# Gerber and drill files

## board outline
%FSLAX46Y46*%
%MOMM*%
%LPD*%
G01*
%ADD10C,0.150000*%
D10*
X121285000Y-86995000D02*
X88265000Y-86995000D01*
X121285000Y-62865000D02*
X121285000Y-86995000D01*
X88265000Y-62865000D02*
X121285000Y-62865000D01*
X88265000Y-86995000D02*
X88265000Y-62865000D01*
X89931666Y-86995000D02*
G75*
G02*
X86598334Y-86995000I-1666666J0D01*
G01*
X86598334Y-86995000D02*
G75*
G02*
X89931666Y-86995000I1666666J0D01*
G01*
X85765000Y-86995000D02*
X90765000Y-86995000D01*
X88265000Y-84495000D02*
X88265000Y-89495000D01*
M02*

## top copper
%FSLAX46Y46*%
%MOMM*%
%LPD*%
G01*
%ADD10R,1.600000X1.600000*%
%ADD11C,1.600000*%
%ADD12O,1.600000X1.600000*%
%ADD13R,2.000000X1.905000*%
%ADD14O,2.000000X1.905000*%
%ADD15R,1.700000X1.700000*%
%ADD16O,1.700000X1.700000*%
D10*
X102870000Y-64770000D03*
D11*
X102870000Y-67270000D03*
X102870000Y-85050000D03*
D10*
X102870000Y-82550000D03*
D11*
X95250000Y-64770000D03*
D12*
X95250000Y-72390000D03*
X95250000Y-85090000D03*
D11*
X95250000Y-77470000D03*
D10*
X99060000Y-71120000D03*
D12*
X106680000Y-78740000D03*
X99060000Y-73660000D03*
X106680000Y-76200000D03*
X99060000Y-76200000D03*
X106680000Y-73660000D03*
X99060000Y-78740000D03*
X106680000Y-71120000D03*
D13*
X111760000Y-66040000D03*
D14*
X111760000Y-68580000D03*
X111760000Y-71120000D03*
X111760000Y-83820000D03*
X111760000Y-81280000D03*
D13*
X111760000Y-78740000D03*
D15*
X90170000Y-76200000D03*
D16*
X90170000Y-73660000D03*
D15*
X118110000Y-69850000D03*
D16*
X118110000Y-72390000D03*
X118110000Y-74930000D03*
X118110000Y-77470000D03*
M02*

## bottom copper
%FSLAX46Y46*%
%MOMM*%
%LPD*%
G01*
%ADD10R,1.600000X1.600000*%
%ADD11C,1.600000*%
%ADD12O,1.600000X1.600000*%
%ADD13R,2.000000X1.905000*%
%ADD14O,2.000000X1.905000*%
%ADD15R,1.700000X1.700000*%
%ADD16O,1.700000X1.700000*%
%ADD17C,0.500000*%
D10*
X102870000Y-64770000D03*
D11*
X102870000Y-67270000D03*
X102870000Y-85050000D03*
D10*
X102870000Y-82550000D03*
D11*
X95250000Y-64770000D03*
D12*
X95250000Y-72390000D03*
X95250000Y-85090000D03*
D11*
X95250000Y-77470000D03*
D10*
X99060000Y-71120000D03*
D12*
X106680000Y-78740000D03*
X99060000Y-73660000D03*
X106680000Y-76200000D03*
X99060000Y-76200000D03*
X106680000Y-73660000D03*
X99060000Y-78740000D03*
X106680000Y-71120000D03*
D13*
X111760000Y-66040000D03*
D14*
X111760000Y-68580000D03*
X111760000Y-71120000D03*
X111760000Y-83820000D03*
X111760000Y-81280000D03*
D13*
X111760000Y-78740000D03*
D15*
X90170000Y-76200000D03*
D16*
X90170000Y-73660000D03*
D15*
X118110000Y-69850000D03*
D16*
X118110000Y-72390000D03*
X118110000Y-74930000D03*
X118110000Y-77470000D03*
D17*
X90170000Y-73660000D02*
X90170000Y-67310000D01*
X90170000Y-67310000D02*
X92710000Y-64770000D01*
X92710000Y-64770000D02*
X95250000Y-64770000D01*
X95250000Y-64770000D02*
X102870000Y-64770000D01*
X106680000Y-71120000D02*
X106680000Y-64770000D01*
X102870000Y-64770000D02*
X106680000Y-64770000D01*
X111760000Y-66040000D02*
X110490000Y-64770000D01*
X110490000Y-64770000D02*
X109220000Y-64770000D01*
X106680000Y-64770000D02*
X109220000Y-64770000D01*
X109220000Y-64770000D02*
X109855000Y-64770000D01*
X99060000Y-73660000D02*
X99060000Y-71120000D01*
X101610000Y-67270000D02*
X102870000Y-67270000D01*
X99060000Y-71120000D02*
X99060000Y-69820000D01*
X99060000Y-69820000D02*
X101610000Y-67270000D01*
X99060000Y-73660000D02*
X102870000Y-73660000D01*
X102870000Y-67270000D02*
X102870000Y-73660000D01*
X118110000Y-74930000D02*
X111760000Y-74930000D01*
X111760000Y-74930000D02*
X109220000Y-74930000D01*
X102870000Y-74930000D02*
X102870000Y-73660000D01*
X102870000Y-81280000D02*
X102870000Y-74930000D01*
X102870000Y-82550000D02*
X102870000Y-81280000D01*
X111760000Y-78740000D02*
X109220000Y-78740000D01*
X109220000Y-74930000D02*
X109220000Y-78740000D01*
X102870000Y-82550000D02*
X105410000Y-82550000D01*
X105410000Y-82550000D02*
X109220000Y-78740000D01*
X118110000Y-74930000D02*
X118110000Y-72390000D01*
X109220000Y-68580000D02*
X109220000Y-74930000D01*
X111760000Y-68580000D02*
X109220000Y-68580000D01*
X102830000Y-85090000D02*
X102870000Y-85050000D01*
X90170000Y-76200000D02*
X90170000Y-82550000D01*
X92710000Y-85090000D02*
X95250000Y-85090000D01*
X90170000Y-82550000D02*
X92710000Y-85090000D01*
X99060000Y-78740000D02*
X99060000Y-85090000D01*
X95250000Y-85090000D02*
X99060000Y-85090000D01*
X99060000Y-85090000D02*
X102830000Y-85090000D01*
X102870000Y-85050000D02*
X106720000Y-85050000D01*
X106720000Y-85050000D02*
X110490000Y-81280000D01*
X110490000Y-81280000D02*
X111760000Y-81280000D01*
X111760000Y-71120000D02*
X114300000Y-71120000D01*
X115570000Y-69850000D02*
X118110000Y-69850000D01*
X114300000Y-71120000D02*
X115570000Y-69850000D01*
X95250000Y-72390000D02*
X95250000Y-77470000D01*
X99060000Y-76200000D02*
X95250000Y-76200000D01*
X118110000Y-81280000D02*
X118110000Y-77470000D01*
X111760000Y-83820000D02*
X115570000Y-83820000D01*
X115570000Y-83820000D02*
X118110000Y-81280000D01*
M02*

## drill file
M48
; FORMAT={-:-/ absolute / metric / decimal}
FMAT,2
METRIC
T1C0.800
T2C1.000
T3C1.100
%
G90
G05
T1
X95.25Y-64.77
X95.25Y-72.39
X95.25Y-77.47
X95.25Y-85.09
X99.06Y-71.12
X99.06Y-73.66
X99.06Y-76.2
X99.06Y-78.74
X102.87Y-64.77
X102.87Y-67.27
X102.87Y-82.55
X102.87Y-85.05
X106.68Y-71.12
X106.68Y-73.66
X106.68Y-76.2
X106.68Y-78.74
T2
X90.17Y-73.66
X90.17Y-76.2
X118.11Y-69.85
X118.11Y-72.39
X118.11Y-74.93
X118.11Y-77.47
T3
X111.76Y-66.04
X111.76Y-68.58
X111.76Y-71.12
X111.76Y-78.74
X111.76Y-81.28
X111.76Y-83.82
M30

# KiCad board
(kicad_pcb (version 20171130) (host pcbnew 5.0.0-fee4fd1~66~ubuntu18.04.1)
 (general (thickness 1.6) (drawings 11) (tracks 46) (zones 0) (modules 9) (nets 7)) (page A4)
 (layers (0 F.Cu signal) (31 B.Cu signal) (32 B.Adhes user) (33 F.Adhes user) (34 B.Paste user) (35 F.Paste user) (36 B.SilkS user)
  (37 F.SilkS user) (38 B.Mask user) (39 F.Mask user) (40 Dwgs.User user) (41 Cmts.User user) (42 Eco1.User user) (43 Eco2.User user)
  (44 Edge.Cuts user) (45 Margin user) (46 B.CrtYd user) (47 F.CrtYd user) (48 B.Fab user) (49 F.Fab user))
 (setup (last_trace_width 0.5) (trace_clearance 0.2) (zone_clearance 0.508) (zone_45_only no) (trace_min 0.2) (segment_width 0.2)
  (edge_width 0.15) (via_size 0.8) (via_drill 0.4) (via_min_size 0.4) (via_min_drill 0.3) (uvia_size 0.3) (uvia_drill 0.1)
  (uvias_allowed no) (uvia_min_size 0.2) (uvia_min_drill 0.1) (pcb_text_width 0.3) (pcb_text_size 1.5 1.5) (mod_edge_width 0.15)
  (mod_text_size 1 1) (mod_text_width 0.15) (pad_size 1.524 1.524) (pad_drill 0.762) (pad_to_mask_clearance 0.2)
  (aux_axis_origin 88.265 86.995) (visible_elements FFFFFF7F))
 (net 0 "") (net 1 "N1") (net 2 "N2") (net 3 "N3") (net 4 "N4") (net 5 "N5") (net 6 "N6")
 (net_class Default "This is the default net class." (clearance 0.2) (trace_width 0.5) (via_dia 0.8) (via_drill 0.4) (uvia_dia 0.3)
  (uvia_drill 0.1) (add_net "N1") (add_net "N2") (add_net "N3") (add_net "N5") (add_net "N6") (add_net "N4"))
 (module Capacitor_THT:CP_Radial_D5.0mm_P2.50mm (layer F.Cu) (at 102.87 64.77 270)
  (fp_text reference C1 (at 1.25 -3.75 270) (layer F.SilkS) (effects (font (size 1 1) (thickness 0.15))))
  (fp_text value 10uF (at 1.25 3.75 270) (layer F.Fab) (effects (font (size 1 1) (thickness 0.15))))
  (pad 1 thru_hole rect (at 0 0 270) (size 1.6 1.6) (drill 0.8) (layers *.Cu *.Mask) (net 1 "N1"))
  (pad 2 thru_hole circle (at 2.5 0 270) (size 1.6 1.6) (drill 0.8) (layers *.Cu *.Mask) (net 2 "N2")))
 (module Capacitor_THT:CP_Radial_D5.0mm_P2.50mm (layer F.Cu) (at 102.87 82.55 270)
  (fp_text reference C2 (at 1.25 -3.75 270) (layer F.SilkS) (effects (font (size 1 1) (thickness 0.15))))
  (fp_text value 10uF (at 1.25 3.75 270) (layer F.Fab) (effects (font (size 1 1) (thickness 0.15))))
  (pad 2 thru_hole circle (at 2.5 0 270) (size 1.6 1.6) (drill 0.8) (layers *.Cu *.Mask) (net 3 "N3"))
  (pad 1 thru_hole rect (at 0 0 270) (size 1.6 1.6) (drill 0.8) (layers *.Cu *.Mask) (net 2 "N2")))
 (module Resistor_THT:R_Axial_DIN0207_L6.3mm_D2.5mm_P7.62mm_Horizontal (layer F.Cu) (at 95.25 64.77 270)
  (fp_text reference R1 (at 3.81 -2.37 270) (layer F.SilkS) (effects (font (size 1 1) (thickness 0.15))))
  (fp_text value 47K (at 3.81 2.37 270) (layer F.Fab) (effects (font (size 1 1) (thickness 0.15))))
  (pad 1 thru_hole circle (at 0 0 270) (size 1.6 1.6) (drill 0.8) (layers *.Cu *.Mask) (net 1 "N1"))
  (pad 2 thru_hole oval (at 7.62 0 270) (size 1.6 1.6) (drill 0.8) (layers *.Cu *.Mask) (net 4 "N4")))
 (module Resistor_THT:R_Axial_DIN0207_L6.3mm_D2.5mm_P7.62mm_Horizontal (layer F.Cu) (at 95.25 77.47 270)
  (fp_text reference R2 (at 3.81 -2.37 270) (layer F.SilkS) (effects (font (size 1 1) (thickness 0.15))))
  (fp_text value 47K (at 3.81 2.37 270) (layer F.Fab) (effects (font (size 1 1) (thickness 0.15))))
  (pad 2 thru_hole oval (at 7.62 0 270) (size 1.6 1.6) (drill 0.8) (layers *.Cu *.Mask) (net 3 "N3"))
  (pad 1 thru_hole circle (at 0 0 270) (size 1.6 1.6) (drill 0.8) (layers *.Cu *.Mask) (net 4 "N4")))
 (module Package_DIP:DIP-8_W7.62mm (layer F.Cu) (at 99.06 71.12)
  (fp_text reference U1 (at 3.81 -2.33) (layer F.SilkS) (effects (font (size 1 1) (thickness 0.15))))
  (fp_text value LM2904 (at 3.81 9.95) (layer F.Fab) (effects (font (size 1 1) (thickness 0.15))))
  (pad 1 thru_hole rect (at 0 0) (size 1.6 1.6) (drill 0.8) (layers *.Cu *.Mask) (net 2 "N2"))
  (pad 5 thru_hole oval (at 7.62 7.62) (size 1.6 1.6) (drill 0.8) (layers *.Cu *.Mask))
  (pad 2 thru_hole oval (at 0 2.54) (size 1.6 1.6) (drill 0.8) (layers *.Cu *.Mask) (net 2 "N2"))
  (pad 6 thru_hole oval (at 7.62 5.08) (size 1.6 1.6) (drill 0.8) (layers *.Cu *.Mask))
  (pad 3 thru_hole oval (at 0 5.08) (size 1.6 1.6) (drill 0.8) (layers *.Cu *.Mask) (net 4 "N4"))
  (pad 7 thru_hole oval (at 7.62 2.54) (size 1.6 1.6) (drill 0.8) (layers *.Cu *.Mask))
  (pad 4 thru_hole oval (at 0 7.62) (size 1.6 1.6) (drill 0.8) (layers *.Cu *.Mask) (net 3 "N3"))
  (pad 8 thru_hole oval (at 7.62 0) (size 1.6 1.6) (drill 0.8) (layers *.Cu *.Mask) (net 1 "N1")))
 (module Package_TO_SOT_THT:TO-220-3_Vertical (layer F.Cu) (at 111.76 66.04 270)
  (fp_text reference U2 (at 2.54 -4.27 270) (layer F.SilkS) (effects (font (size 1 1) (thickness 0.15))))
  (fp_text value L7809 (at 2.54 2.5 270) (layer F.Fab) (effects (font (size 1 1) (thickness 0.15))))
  (pad 1 thru_hole rect (at 0 0 270) (size 1.905 2) (drill 1.1) (layers *.Cu *.Mask) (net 1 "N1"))
  (pad 2 thru_hole oval (at 2.54 0 270) (size 1.905 2) (drill 1.1) (layers *.Cu *.Mask) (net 2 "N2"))
  (pad 3 thru_hole oval (at 5.08 0 270) (size 1.905 2) (drill 1.1) (layers *.Cu *.Mask) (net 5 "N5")))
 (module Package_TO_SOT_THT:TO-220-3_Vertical (layer F.Cu) (at 111.76 78.74 270)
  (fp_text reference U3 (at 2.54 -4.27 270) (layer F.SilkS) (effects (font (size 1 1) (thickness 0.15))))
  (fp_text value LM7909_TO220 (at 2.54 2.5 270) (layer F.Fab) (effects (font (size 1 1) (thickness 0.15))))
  (pad 3 thru_hole oval (at 5.08 0 270) (size 1.905 2) (drill 1.1) (layers *.Cu *.Mask) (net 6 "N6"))
  (pad 2 thru_hole oval (at 2.54 0 270) (size 1.905 2) (drill 1.1) (layers *.Cu *.Mask) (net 3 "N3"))
  (pad 1 thru_hole rect (at 0 0 270) (size 1.905 2) (drill 1.1) (layers *.Cu *.Mask) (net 2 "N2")))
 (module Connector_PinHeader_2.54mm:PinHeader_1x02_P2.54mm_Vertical (layer F.Cu) (at 90.17 76.2 180)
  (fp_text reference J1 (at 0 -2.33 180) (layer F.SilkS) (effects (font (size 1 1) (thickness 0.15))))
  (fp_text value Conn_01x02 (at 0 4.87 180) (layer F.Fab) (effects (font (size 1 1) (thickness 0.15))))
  (pad 1 thru_hole rect (at 0 0 180) (size 1.7 1.7) (drill 1) (layers *.Cu *.Mask) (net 3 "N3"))
  (pad 2 thru_hole oval (at 0 2.54 180) (size 1.7 1.7) (drill 1) (layers *.Cu *.Mask) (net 1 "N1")))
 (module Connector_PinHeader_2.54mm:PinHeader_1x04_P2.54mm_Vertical (layer F.Cu) (at 118.11 69.85)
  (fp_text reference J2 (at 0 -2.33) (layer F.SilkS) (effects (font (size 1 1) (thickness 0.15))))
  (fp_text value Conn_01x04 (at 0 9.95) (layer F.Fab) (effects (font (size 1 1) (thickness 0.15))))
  (pad 1 thru_hole rect (at 0 0) (size 1.7 1.7) (drill 1) (layers *.Cu *.Mask) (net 5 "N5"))
  (pad 2 thru_hole oval (at 0 2.54) (size 1.7 1.7) (drill 1) (layers *.Cu *.Mask) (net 2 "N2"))
  (pad 3 thru_hole oval (at 0 5.08) (size 1.7 1.7) (drill 1) (layers *.Cu *.Mask) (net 2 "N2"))
  (pad 4 thru_hole oval (at 0 7.62) (size 1.7 1.7) (drill 1) (layers *.Cu *.Mask) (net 6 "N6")))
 (gr_line (start 121.285 86.995) (end 88.265 86.995) (layer Edge.Cuts) (width 0.15))
 (gr_line (start 121.285 62.865) (end 121.285 86.995) (layer Edge.Cuts) (width 0.15))
 (gr_line (start 88.265 62.865) (end 121.285 62.865) (layer Edge.Cuts) (width 0.15))
 (gr_line (start 88.265 86.995) (end 88.265 62.865) (layer Edge.Cuts) (width 0.15))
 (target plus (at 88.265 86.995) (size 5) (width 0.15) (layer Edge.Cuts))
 (segment (start 90.17 73.66) (end 90.17 67.31) (width 0.5) (layer B.Cu) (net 1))
 (segment (start 90.17 67.31) (end 92.71 64.77) (width 0.5) (layer B.Cu) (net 1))
 (segment (start 92.71 64.77) (end 95.25 64.77) (width 0.5) (layer B.Cu) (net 1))
 (segment (start 95.25 64.77) (end 102.87 64.77) (width 0.5) (layer B.Cu) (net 1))
 (segment (start 106.68 71.12) (end 106.68 64.77) (width 0.5) (layer B.Cu) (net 1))
 (segment (start 102.87 64.77) (end 106.68 64.77) (width 0.5) (layer B.Cu) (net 1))
 (segment (start 111.76 66.04) (end 110.49 64.77) (width 0.5) (layer B.Cu) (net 1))
 (segment (start 110.49 64.77) (end 109.22 64.77) (width 0.5) (layer B.Cu) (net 1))
 (segment (start 106.68 64.77) (end 109.22 64.77) (width 0.5) (layer B.Cu) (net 1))
 (segment (start 109.22 64.77) (end 109.855 64.77) (width 0.5) (layer B.Cu) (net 1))
 (segment (start 99.06 73.66) (end 99.06 71.12) (width 0.5) (layer B.Cu) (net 2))
 (segment (start 101.61 67.27) (end 102.87 67.27) (width 0.5) (layer B.Cu) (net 2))
 (segment (start 99.06 71.12) (end 99.06 69.82) (width 0.5) (layer B.Cu) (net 2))
 (segment (start 99.06 69.82) (end 101.61 67.27) (width 0.5) (layer B.Cu) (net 2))
 (segment (start 99.06 73.66) (end 102.87 73.66) (width 0.5) (layer B.Cu) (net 2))
 (segment (start 102.87 67.27) (end 102.87 73.66) (width 0.5) (layer B.Cu) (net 2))
 (segment (start 118.11 74.93) (end 111.76 74.93) (width 0.5) (layer B.Cu) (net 2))
 (segment (start 111.76 74.93) (end 109.22 74.93) (width 0.5) (layer B.Cu) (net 2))
 (segment (start 102.87 74.93) (end 102.87 73.66) (width 0.5) (layer B.Cu) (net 2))
 (segment (start 102.87 81.28) (end 102.87 74.93) (width 0.5) (layer B.Cu) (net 2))
 (segment (start 102.87 82.55) (end 102.87 81.28) (width 0.5) (layer B.Cu) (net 2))
 (segment (start 111.76 78.74) (end 109.22 78.74) (width 0.5) (layer B.Cu) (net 2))
 (segment (start 109.22 74.93) (end 109.22 78.74) (width 0.5) (layer B.Cu) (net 2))
 (segment (start 102.87 82.55) (end 105.41 82.55) (width 0.5) (layer B.Cu) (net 2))
 (segment (start 105.41 82.55) (end 109.22 78.74) (width 0.5) (layer B.Cu) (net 2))
 (segment (start 118.11 74.93) (end 118.11 72.39) (width 0.5) (layer B.Cu) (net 2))
 (segment (start 109.22 68.58) (end 109.22 74.93) (width 0.5) (layer B.Cu) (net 2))
 (segment (start 111.76 68.58) (end 109.22 68.58) (width 0.5) (layer B.Cu) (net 2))
 (segment (start 102.83 85.09) (end 102.87 85.05) (width 0.5) (layer B.Cu) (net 3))
 (segment (start 90.17 76.2) (end 90.17 82.55) (width 0.5) (layer B.Cu) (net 3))
 (segment (start 92.71 85.09) (end 95.25 85.09) (width 0.5) (layer B.Cu) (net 3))
 (segment (start 90.17 82.55) (end 92.71 85.09) (width 0.5) (layer B.Cu) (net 3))
 (segment (start 99.06 78.74) (end 99.06 85.09) (width 0.5) (layer B.Cu) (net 3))
 (segment (start 95.25 85.09) (end 99.06 85.09) (width 0.5) (layer B.Cu) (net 3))
 (segment (start 99.06 85.09) (end 102.83 85.09) (width 0.5) (layer B.Cu) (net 3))
 (segment (start 102.87 85.05) (end 106.72 85.05) (width 0.5) (layer B.Cu) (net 3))
 (segment (start 106.72 85.05) (end 110.49 81.28) (width 0.5) (layer B.Cu) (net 3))
 (segment (start 110.49 81.28) (end 111.76 81.28) (width 0.5) (layer B.Cu) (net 3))
 (segment (start 111.76 71.12) (end 114.3 71.12) (width 0.5) (layer B.Cu) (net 5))
 (segment (start 115.57 69.85) (end 118.11 69.85) (width 0.5) (layer B.Cu) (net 5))
 (segment (start 114.3 71.12) (end 115.57 69.85) (width 0.5) (layer B.Cu) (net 5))
 (segment (start 95.25 72.39) (end 95.25 77.47) (width 0.5) (layer B.Cu) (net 4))
 (segment (start 99.06 76.2) (end 95.25 76.2) (width 0.5) (layer B.Cu) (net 4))
 (segment (start 118.11 81.28) (end 118.11 77.47) (width 0.5) (layer B.Cu) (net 6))
 (segment (start 111.76 83.82) (end 115.57 83.82) (width 0.5) (layer B.Cu) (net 6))
 (segment (start 115.57 83.82) (end 118.11 81.28) (width 0.5) (layer B.Cu) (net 6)))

